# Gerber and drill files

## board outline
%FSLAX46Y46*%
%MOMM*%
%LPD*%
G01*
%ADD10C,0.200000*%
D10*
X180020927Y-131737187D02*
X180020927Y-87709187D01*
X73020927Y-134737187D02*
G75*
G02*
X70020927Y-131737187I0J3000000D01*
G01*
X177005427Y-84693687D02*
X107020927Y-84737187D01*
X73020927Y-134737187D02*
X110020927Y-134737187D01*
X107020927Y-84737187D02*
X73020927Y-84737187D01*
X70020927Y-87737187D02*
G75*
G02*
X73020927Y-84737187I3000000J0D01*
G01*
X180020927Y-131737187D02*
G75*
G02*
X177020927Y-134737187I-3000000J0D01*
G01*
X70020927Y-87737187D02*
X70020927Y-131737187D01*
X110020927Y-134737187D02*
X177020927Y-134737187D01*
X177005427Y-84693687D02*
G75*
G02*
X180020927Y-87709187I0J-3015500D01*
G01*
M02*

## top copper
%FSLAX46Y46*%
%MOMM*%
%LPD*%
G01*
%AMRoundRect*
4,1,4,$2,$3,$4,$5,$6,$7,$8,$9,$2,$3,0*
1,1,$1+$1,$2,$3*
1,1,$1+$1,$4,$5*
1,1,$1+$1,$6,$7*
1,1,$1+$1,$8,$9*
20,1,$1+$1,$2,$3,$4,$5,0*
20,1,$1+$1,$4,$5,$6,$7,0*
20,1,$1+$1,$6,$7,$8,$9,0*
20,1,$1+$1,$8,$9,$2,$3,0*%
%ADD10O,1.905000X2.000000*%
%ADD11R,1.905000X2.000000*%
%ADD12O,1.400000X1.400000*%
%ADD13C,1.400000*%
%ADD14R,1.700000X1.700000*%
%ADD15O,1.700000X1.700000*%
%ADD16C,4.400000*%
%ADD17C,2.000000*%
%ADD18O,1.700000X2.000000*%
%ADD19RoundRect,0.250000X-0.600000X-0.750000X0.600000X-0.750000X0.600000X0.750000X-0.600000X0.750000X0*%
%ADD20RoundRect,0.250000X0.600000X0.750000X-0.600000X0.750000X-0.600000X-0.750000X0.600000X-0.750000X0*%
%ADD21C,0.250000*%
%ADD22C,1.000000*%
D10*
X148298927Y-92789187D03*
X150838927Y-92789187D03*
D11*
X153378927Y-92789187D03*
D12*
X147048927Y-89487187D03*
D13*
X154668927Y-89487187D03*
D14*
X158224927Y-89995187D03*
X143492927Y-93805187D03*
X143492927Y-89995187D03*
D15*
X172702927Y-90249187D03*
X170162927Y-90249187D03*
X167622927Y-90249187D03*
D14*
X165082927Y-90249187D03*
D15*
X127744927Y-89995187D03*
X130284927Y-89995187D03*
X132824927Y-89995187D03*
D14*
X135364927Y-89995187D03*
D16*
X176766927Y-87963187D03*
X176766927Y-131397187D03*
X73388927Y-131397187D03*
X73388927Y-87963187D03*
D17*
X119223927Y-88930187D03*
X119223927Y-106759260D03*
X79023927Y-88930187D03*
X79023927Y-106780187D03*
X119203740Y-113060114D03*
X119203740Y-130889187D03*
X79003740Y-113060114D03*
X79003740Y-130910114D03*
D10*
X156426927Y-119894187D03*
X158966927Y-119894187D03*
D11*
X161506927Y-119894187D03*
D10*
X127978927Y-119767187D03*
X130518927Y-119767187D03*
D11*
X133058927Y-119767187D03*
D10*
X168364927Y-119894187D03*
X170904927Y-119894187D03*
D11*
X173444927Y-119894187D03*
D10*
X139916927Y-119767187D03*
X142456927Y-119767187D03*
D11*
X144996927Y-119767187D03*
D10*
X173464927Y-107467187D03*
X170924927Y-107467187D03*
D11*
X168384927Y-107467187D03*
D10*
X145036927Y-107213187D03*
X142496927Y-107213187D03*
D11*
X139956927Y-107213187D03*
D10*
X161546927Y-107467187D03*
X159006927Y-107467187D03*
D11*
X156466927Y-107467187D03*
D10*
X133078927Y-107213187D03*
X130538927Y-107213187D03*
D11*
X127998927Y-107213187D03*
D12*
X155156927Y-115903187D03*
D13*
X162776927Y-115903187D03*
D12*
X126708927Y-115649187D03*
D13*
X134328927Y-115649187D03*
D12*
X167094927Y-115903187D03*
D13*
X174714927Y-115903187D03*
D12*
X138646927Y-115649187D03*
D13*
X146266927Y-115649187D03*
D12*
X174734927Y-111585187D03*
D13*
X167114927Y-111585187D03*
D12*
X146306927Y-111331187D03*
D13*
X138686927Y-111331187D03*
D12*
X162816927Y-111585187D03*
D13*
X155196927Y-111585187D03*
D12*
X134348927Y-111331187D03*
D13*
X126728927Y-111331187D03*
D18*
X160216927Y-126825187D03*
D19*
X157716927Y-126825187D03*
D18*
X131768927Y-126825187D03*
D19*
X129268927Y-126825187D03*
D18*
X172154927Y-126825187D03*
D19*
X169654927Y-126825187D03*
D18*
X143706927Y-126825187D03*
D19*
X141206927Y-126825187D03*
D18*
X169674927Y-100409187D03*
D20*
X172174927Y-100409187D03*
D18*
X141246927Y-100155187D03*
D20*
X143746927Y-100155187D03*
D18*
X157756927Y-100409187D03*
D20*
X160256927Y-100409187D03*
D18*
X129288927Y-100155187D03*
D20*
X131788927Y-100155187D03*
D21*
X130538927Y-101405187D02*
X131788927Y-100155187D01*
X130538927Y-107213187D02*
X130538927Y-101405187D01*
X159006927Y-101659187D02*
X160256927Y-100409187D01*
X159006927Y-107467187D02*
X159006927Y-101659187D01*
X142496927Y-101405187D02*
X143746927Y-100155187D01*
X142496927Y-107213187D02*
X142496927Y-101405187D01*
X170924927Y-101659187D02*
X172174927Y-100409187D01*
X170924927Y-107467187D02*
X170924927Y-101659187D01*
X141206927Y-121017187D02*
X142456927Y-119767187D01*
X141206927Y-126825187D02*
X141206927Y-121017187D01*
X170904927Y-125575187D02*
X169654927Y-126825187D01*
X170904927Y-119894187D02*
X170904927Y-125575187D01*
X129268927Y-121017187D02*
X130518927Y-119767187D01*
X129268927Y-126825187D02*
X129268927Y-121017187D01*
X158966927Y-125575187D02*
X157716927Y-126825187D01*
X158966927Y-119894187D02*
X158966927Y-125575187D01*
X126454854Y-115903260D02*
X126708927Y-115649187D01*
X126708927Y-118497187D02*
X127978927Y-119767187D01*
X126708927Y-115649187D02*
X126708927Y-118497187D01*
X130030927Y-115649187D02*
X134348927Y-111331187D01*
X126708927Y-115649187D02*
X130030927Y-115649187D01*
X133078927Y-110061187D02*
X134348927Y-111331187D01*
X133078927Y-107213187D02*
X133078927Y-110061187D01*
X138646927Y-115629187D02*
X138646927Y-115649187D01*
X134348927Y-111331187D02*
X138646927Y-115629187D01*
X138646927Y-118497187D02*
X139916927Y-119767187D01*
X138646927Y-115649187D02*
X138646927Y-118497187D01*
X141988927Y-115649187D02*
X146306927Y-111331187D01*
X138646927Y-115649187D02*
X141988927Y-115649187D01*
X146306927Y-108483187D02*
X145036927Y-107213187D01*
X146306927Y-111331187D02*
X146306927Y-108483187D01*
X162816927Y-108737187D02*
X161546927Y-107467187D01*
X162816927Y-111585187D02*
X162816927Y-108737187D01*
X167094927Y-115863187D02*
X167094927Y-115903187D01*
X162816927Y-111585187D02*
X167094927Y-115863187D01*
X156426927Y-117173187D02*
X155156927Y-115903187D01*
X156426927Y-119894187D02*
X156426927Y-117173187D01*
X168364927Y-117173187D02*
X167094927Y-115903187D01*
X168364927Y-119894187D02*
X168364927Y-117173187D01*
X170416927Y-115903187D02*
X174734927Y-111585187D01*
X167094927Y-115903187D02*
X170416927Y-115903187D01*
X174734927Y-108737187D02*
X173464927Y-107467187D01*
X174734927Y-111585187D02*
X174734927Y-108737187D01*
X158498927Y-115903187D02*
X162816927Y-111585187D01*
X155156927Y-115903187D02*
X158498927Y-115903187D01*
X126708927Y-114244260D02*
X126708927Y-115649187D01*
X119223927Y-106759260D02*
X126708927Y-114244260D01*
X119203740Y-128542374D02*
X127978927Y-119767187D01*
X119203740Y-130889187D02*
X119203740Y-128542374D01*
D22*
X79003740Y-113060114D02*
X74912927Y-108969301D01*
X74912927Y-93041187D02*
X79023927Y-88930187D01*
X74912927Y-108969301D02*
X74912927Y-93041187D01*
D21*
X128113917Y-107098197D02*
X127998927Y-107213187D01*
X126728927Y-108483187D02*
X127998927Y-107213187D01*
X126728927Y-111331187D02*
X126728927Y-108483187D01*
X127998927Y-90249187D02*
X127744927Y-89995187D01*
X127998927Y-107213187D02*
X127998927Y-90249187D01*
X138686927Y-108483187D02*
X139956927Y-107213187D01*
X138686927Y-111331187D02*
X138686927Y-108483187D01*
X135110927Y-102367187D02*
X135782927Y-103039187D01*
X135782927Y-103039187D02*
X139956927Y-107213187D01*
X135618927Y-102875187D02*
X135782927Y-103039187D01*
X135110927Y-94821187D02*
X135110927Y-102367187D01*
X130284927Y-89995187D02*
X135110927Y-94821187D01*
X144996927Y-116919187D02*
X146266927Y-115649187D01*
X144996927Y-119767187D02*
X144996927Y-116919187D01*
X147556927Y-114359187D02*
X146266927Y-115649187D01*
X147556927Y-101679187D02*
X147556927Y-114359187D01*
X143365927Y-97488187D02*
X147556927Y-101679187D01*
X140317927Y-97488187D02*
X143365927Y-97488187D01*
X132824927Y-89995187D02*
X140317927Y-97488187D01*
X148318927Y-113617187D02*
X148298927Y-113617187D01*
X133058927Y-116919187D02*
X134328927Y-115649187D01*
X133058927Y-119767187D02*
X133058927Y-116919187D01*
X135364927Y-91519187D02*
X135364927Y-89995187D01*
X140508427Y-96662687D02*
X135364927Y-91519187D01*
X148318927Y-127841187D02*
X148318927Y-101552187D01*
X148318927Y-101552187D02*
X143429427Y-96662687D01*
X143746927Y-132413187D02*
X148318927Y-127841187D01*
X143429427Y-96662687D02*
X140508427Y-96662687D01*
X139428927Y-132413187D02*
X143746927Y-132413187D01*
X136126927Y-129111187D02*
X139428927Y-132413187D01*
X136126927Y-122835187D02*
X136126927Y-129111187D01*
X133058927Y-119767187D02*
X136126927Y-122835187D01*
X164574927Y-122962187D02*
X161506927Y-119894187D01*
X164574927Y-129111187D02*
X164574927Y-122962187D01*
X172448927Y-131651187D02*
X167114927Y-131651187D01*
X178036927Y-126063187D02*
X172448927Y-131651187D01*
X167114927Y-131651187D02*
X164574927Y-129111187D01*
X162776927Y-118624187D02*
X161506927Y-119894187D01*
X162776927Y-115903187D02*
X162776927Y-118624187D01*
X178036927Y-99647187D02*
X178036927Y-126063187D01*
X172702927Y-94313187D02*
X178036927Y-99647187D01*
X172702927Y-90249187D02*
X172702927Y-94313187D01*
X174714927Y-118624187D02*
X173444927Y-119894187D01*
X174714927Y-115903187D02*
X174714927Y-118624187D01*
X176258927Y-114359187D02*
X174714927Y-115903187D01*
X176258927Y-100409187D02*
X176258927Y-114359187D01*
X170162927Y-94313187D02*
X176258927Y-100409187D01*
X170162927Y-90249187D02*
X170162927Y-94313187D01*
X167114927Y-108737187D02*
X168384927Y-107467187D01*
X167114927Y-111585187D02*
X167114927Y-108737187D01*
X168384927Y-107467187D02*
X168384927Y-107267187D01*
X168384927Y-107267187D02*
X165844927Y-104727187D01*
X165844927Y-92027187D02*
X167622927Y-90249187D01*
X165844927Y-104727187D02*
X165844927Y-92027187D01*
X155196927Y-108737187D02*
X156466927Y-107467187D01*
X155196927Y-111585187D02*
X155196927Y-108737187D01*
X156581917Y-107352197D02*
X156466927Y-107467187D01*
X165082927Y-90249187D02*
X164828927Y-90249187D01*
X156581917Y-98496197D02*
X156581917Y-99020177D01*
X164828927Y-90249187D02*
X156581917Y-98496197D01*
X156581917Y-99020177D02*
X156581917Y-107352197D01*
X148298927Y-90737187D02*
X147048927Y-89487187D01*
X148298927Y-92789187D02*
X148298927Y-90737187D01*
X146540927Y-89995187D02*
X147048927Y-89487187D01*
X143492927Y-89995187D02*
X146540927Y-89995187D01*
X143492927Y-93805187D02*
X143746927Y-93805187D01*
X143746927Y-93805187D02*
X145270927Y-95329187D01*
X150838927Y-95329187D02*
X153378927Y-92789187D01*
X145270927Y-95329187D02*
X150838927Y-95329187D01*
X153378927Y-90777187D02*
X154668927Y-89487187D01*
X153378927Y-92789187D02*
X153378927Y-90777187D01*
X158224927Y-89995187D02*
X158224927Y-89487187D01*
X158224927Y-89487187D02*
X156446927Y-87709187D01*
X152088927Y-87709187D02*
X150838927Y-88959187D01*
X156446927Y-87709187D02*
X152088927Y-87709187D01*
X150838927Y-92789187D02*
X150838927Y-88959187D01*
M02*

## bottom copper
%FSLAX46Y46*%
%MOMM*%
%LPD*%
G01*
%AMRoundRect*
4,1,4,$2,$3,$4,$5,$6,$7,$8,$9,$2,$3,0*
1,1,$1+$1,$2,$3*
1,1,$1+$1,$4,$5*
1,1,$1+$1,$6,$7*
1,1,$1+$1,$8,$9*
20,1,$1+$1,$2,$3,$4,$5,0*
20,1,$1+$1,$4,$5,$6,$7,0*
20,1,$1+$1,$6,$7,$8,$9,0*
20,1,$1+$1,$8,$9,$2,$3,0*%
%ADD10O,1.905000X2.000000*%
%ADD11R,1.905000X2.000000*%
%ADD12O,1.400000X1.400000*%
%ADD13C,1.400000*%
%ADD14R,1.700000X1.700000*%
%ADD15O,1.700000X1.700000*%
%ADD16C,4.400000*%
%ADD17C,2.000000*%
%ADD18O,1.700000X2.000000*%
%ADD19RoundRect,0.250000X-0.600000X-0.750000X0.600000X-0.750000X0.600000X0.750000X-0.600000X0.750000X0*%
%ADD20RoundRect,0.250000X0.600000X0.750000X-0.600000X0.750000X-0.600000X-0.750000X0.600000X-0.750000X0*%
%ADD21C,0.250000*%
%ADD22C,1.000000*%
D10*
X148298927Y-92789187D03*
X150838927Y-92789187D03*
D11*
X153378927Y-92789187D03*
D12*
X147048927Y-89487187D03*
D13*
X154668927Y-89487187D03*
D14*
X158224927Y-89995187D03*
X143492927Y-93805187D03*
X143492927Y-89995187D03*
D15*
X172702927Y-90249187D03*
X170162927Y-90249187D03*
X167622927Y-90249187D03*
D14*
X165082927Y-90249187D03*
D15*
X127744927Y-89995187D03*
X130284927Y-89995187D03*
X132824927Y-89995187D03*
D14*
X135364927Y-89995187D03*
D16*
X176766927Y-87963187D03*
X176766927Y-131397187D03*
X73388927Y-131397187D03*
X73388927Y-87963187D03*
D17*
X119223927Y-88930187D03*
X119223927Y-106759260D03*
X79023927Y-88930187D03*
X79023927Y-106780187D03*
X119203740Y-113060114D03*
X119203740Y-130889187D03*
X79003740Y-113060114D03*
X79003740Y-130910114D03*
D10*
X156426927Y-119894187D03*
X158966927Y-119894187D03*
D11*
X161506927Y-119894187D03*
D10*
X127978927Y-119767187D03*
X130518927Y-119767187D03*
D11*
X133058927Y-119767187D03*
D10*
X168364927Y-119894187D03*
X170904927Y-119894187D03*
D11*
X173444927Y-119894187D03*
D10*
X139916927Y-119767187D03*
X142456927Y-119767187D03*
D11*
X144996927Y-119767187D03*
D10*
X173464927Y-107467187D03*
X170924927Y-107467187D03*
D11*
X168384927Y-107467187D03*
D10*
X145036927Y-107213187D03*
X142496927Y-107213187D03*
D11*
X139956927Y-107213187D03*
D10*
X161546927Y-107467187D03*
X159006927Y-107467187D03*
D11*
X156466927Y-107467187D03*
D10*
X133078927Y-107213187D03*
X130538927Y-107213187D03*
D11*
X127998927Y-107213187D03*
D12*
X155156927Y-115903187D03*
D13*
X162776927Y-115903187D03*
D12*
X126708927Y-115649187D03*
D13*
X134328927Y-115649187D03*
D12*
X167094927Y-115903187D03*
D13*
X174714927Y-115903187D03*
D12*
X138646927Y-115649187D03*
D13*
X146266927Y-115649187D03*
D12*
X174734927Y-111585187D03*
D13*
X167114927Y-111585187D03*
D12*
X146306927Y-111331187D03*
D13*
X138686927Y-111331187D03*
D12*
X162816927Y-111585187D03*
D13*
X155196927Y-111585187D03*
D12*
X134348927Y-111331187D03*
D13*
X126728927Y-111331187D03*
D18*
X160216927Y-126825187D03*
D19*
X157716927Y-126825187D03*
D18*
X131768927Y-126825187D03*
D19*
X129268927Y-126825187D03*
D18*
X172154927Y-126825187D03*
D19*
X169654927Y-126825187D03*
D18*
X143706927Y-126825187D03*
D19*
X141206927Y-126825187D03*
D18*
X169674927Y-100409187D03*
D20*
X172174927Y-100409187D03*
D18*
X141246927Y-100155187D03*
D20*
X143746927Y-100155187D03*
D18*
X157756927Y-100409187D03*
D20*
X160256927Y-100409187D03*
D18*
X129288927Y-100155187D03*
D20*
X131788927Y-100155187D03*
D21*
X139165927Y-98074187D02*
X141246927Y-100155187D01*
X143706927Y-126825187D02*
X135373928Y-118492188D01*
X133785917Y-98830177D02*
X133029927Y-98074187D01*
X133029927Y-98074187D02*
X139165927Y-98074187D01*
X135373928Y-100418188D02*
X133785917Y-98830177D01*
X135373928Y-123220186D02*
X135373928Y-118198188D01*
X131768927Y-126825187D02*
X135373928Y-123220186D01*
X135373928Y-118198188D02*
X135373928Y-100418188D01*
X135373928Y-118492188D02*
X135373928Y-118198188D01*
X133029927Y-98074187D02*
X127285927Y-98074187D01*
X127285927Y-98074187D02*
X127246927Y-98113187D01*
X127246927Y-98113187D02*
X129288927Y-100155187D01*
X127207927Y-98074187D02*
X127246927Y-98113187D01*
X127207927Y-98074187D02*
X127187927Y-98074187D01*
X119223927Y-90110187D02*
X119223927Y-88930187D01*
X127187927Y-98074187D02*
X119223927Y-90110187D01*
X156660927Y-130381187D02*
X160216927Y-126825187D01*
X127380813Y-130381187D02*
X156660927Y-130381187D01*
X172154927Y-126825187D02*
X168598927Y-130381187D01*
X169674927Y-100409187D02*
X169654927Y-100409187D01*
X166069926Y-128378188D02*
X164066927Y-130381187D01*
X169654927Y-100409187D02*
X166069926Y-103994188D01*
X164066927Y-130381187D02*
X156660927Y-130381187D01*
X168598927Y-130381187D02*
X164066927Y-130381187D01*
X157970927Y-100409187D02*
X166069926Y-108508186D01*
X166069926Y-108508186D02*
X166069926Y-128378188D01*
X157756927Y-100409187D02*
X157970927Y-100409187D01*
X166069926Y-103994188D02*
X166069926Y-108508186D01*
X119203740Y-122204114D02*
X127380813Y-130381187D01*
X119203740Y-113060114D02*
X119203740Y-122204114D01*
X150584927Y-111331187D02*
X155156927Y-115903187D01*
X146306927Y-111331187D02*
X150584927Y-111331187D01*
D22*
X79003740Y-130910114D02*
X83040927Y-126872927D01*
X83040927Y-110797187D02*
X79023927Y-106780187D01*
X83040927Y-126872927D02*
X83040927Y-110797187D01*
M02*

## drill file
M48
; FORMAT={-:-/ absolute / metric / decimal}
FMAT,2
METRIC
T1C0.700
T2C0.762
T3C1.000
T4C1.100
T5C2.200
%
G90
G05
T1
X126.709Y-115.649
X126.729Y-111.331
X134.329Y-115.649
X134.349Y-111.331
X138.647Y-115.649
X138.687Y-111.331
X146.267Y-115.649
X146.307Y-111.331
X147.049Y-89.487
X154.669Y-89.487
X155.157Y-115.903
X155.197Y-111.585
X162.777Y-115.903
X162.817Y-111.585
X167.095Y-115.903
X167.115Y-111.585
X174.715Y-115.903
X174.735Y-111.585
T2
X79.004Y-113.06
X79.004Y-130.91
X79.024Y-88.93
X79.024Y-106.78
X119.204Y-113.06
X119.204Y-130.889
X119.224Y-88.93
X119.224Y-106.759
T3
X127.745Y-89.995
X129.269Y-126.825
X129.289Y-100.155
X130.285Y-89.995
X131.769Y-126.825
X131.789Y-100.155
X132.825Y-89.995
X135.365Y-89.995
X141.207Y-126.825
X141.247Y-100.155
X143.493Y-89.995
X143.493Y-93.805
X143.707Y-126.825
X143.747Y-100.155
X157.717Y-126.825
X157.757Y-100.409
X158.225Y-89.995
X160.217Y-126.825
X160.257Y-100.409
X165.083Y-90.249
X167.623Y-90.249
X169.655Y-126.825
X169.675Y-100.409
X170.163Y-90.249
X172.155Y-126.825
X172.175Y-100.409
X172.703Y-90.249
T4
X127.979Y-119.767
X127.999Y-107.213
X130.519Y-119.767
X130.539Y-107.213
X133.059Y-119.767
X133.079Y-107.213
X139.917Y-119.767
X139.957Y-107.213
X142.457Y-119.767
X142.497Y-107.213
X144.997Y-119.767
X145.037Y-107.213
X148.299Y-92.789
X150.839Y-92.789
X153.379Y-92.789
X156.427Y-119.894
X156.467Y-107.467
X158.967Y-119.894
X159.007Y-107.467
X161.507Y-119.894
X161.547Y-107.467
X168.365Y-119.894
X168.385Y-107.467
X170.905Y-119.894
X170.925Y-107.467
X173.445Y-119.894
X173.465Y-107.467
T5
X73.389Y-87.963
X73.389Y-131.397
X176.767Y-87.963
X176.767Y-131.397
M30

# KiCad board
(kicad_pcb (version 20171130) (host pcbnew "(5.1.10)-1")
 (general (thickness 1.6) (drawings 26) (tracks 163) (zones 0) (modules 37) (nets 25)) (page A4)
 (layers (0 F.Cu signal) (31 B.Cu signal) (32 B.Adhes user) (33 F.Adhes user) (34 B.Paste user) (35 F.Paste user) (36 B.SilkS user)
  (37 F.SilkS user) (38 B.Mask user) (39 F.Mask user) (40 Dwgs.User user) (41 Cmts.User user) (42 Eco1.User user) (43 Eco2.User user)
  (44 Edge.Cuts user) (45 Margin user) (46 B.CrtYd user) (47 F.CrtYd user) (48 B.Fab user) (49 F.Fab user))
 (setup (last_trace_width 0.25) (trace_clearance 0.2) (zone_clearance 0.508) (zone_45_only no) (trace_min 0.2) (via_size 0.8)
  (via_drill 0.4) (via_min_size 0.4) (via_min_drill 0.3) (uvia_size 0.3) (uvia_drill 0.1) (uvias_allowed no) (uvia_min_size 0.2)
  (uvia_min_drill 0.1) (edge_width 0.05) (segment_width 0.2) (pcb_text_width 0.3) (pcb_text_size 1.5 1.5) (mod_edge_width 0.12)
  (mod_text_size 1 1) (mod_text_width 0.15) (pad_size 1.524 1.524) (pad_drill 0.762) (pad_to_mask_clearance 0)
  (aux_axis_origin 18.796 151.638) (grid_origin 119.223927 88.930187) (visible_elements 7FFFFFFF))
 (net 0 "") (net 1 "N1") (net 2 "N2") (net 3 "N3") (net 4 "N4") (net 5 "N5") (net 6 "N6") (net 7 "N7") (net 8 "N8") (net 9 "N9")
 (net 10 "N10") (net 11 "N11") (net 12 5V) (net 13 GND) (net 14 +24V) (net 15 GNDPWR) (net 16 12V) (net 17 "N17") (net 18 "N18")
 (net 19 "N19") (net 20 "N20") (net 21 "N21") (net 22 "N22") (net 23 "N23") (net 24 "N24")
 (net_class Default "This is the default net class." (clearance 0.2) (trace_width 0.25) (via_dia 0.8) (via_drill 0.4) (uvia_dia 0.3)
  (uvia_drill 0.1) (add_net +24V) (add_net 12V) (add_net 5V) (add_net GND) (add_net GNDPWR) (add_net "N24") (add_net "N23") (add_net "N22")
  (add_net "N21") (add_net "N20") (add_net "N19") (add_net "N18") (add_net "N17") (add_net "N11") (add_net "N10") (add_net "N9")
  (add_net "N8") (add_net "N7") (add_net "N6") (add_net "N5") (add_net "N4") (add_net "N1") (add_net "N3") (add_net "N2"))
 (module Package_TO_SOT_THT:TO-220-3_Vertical (layer F.Cu) (at 153.378927 92.789187 180)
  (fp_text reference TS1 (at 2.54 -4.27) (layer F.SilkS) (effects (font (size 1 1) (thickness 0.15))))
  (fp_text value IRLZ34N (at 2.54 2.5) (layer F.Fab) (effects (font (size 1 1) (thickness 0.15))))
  (pad 3 thru_hole oval (at 5.08 0 180) (size 1.905 2) (drill 1.1) (layers *.Cu *.Mask) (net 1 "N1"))
  (pad 2 thru_hole oval (at 2.54 0 180) (size 1.905 2) (drill 1.1) (layers *.Cu *.Mask) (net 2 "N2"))
  (pad 1 thru_hole rect (at 0 0 180) (size 1.905 2) (drill 1.1) (layers *.Cu *.Mask) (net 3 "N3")))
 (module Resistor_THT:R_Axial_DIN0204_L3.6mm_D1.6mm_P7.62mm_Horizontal (layer F.Cu) (at 154.668927 89.487187 180)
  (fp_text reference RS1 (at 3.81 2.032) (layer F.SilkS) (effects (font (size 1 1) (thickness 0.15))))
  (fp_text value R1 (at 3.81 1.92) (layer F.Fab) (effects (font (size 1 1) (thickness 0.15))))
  (pad 2 thru_hole oval (at 7.62 0 180) (size 1.4 1.4) (drill 0.7) (layers *.Cu *.Mask) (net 1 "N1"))
  (pad 1 thru_hole circle (at 0 0 180) (size 1.4 1.4) (drill 0.7) (layers *.Cu *.Mask) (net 3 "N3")))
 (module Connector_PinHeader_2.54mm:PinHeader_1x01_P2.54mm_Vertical (layer F.Cu) (at 158.224927 89.995187 180)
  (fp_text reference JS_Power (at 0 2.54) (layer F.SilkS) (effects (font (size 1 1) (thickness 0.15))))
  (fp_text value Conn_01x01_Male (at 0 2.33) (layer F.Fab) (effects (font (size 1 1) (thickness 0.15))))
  (pad 1 thru_hole rect (at 0 0 180) (size 1.7 1.7) (drill 1) (layers *.Cu *.Mask) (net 2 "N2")))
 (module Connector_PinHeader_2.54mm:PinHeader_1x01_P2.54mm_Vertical (layer F.Cu) (at 143.492927 93.805187 180)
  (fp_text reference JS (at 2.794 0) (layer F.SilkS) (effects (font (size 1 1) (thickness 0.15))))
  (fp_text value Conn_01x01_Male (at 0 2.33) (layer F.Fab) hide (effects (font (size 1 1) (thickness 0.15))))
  (pad 1 thru_hole rect (at 0 0 180) (size 1.7 1.7) (drill 1) (layers *.Cu *.Mask) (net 3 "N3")))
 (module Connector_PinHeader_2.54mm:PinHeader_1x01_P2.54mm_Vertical (layer F.Cu) (at 143.492927 89.995187 180)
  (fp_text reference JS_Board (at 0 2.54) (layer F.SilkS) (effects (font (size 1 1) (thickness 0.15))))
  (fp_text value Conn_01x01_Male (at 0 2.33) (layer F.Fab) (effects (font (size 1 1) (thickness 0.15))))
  (pad 1 thru_hole rect (at 0 0 180) (size 1.7 1.7) (drill 1) (layers *.Cu *.Mask) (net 1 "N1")))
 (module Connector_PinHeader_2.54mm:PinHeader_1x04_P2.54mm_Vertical (layer F.Cu) (at 165.082927 90.249187 90)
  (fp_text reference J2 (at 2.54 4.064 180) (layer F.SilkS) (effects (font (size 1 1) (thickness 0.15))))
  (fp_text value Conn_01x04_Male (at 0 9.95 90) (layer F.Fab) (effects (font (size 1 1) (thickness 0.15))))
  (pad 4 thru_hole oval (at 0 7.62 90) (size 1.7 1.7) (drill 1) (layers *.Cu *.Mask) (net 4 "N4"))
  (pad 3 thru_hole oval (at 0 5.08 90) (size 1.7 1.7) (drill 1) (layers *.Cu *.Mask) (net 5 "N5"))
  (pad 2 thru_hole oval (at 0 2.54 90) (size 1.7 1.7) (drill 1) (layers *.Cu *.Mask) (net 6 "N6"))
  (pad 1 thru_hole rect (at 0 0 90) (size 1.7 1.7) (drill 1) (layers *.Cu *.Mask) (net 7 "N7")))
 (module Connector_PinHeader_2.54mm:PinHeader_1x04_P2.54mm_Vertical (layer F.Cu) (at 135.364927 89.995187 270)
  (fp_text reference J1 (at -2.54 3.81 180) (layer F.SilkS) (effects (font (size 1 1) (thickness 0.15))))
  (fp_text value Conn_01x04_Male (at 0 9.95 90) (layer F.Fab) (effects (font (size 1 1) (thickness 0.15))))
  (pad 4 thru_hole oval (at 0 7.62 270) (size 1.7 1.7) (drill 1) (layers *.Cu *.Mask) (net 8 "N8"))
  (pad 3 thru_hole oval (at 0 5.08 270) (size 1.7 1.7) (drill 1) (layers *.Cu *.Mask) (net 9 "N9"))
  (pad 2 thru_hole oval (at 0 2.54 270) (size 1.7 1.7) (drill 1) (layers *.Cu *.Mask) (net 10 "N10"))
  (pad 1 thru_hole rect (at 0 0 270) (size 1.7 1.7) (drill 1) (layers *.Cu *.Mask) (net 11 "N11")))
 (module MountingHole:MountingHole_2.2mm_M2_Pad (layer F.Cu) (at 176.766927 87.963187)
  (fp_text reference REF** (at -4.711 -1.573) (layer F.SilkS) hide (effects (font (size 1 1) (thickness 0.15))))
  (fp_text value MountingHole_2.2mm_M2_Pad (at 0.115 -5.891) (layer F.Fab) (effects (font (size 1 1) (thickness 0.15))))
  (pad 1 thru_hole circle (at 0 0) (size 4.4 4.4) (drill 2.2) (layers *.Cu *.Mask)))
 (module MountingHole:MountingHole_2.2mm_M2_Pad (layer F.Cu) (at 176.766927 131.397187)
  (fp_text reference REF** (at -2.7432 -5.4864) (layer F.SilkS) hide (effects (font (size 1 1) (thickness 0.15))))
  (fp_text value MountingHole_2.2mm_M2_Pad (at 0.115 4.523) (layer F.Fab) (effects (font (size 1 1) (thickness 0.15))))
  (pad 1 thru_hole circle (at 0 0) (size 4.4 4.4) (drill 2.2) (layers *.Cu *.Mask)))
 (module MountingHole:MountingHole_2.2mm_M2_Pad (layer F.Cu) (at 73.388927 131.397187)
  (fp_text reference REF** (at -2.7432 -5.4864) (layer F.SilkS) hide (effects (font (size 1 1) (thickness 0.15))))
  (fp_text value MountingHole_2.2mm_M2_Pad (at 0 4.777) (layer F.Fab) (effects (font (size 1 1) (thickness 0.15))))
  (pad 1 thru_hole circle (at 0 0) (size 4.4 4.4) (drill 2.2) (layers *.Cu *.Mask)))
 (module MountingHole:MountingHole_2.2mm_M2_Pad (layer F.Cu) (at 73.388927 87.963187)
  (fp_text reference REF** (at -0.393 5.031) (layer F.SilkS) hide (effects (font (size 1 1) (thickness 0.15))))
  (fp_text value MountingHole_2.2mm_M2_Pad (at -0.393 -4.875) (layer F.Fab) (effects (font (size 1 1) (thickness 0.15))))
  (pad 1 thru_hole circle (at 0 0) (size 4.4 4.4) (drill 2.2) (layers *.Cu *.Mask)))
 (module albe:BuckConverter (layer F.Cu) (at 99.825114 97.86926 270)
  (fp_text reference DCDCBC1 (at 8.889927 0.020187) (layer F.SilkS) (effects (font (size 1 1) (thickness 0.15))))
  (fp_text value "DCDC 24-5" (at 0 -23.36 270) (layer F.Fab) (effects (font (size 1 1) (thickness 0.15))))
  (pad 4 thru_hole circle (at -8.939073 -19.398813 270) (size 2 2) (drill 0.762) (layers *.Cu *.Mask) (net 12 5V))
  (pad 3 thru_hole circle (at 8.89 -19.398813 270) (size 2 2) (drill 0.762) (layers *.Cu *.Mask) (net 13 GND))
  (pad 2 thru_hole circle (at -8.939073 20.801187 270) (size 2 2) (drill 0.762) (layers *.Cu *.Mask) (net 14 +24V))
  (pad 1 thru_hole circle (at 8.910927 20.801187 270) (size 2 2) (drill 0.762) (layers *.Cu *.Mask) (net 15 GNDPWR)))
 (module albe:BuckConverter (layer F.Cu) (at 99.804927 121.999187 270)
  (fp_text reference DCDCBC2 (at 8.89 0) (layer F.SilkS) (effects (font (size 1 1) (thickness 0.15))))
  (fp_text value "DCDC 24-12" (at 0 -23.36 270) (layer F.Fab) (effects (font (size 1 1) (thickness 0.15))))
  (pad 4 thru_hole circle (at -8.939073 -19.398813 270) (size 2 2) (drill 0.762) (layers *.Cu *.Mask) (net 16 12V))
  (pad 3 thru_hole circle (at 8.89 -19.398813 270) (size 2 2) (drill 0.762) (layers *.Cu *.Mask) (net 13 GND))
  (pad 2 thru_hole circle (at -8.939073 20.801187 270) (size 2 2) (drill 0.762) (layers *.Cu *.Mask) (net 14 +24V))
  (pad 1 thru_hole circle (at 8.910927 20.801187 270) (size 2 2) (drill 0.762) (layers *.Cu *.Mask) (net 15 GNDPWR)))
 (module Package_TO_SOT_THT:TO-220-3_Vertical (layer F.Cu) (at 161.506927 119.894187 180)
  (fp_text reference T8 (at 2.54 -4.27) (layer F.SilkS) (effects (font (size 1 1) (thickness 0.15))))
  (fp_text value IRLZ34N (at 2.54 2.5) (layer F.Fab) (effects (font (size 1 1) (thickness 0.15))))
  (pad 3 thru_hole oval (at 5.08 0 180) (size 1.905 2) (drill 1.1) (layers *.Cu *.Mask) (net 13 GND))
  (pad 2 thru_hole oval (at 2.54 0 180) (size 1.905 2) (drill 1.1) (layers *.Cu *.Mask) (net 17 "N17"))
  (pad 1 thru_hole rect (at 0 0 180) (size 1.905 2) (drill 1.1) (layers *.Cu *.Mask) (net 4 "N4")))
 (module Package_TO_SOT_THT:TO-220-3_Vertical (layer F.Cu) (at 133.058927 119.767187 180)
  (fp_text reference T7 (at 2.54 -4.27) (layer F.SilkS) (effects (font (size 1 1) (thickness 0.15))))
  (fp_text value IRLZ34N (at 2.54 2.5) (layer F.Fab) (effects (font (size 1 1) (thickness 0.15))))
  (pad 3 thru_hole oval (at 5.08 0 180) (size 1.905 2) (drill 1.1) (layers *.Cu *.Mask) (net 13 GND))
  (pad 2 thru_hole oval (at 2.54 0 180) (size 1.905 2) (drill 1.1) (layers *.Cu *.Mask) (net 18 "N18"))
  (pad 1 thru_hole rect (at 0 0 180) (size 1.905 2) (drill 1.1) (layers *.Cu *.Mask) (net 11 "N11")))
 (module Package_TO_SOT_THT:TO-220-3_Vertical (layer F.Cu) (at 173.444927 119.894187 180)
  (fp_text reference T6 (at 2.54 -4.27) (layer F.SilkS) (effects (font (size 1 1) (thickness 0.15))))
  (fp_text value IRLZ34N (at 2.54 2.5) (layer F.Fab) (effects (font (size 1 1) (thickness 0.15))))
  (pad 3 thru_hole oval (at 5.08 0 180) (size 1.905 2) (drill 1.1) (layers *.Cu *.Mask) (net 13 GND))
  (pad 2 thru_hole oval (at 2.54 0 180) (size 1.905 2) (drill 1.1) (layers *.Cu *.Mask) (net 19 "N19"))
  (pad 1 thru_hole rect (at 0 0 180) (size 1.905 2) (drill 1.1) (layers *.Cu *.Mask) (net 5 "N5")))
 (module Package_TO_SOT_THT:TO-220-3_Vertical (layer F.Cu) (at 144.996927 119.767187 180)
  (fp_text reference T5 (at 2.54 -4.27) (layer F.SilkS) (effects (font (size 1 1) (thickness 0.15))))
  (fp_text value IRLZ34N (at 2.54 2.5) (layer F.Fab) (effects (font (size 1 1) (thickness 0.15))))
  (pad 3 thru_hole oval (at 5.08 0 180) (size 1.905 2) (drill 1.1) (layers *.Cu *.Mask) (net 13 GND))
  (pad 2 thru_hole oval (at 2.54 0 180) (size 1.905 2) (drill 1.1) (layers *.Cu *.Mask) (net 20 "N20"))
  (pad 1 thru_hole rect (at 0 0 180) (size 1.905 2) (drill 1.1) (layers *.Cu *.Mask) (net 10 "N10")))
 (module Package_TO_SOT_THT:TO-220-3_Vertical (layer F.Cu) (at 168.384927 107.467187)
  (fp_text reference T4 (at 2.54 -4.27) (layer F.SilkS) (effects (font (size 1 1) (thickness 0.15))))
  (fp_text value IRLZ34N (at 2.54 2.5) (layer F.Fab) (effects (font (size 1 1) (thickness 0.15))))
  (pad 3 thru_hole oval (at 5.08 0) (size 1.905 2) (drill 1.1) (layers *.Cu *.Mask) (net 13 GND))
  (pad 2 thru_hole oval (at 2.54 0) (size 1.905 2) (drill 1.1) (layers *.Cu *.Mask) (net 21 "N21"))
  (pad 1 thru_hole rect (at 0 0) (size 1.905 2) (drill 1.1) (layers *.Cu *.Mask) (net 6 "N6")))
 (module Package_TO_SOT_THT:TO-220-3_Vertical (layer F.Cu) (at 139.956927 107.213187)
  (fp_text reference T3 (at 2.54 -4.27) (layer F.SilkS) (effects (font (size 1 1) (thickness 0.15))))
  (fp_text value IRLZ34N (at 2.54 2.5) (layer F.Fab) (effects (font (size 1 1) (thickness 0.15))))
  (pad 3 thru_hole oval (at 5.08 0) (size 1.905 2) (drill 1.1) (layers *.Cu *.Mask) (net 13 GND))
  (pad 2 thru_hole oval (at 2.54 0) (size 1.905 2) (drill 1.1) (layers *.Cu *.Mask) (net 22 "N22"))
  (pad 1 thru_hole rect (at 0 0) (size 1.905 2) (drill 1.1) (layers *.Cu *.Mask) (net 9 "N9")))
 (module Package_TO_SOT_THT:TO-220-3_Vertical (layer F.Cu) (at 156.466927 107.467187)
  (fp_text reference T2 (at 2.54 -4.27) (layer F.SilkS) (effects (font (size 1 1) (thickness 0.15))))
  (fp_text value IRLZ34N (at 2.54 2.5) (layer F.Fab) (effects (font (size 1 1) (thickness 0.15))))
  (pad 3 thru_hole oval (at 5.08 0) (size 1.905 2) (drill 1.1) (layers *.Cu *.Mask) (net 13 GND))
  (pad 2 thru_hole oval (at 2.54 0) (size 1.905 2) (drill 1.1) (layers *.Cu *.Mask) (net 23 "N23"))
  (pad 1 thru_hole rect (at 0 0) (size 1.905 2) (drill 1.1) (layers *.Cu *.Mask) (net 7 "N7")))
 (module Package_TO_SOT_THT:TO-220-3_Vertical (layer F.Cu) (at 127.998927 107.213187)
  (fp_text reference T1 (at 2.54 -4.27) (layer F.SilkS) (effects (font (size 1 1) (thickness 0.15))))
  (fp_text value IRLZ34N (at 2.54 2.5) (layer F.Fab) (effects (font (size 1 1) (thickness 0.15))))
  (pad 3 thru_hole oval (at 5.08 0) (size 1.905 2) (drill 1.1) (layers *.Cu *.Mask) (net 13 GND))
  (pad 2 thru_hole oval (at 2.54 0) (size 1.905 2) (drill 1.1) (layers *.Cu *.Mask) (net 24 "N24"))
  (pad 1 thru_hole rect (at 0 0) (size 1.905 2) (drill 1.1) (layers *.Cu *.Mask) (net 8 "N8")))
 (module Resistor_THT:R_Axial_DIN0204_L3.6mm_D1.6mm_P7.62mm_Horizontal (layer F.Cu) (at 162.776927 115.903187 180)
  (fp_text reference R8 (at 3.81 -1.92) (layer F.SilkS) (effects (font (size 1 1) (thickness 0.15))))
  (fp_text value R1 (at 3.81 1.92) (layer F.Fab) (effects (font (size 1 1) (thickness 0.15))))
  (pad 2 thru_hole oval (at 7.62 0 180) (size 1.4 1.4) (drill 0.7) (layers *.Cu *.Mask) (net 13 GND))
  (pad 1 thru_hole circle (at 0 0 180) (size 1.4 1.4) (drill 0.7) (layers *.Cu *.Mask) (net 4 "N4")))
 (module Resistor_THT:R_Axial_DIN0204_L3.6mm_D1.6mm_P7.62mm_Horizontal (layer F.Cu) (at 134.328927 115.649187 180)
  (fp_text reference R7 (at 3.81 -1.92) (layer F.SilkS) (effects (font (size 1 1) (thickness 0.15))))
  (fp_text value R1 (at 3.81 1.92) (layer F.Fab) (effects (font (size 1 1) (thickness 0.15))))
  (pad 2 thru_hole oval (at 7.62 0 180) (size 1.4 1.4) (drill 0.7) (layers *.Cu *.Mask) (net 13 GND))
  (pad 1 thru_hole circle (at 0 0 180) (size 1.4 1.4) (drill 0.7) (layers *.Cu *.Mask) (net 11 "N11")))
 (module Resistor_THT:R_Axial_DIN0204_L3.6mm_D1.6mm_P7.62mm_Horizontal (layer F.Cu) (at 174.714927 115.903187 180)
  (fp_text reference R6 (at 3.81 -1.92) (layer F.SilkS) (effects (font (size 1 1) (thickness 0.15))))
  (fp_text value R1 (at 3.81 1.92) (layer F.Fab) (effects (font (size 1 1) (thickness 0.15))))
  (pad 2 thru_hole oval (at 7.62 0 180) (size 1.4 1.4) (drill 0.7) (layers *.Cu *.Mask) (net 13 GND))
  (pad 1 thru_hole circle (at 0 0 180) (size 1.4 1.4) (drill 0.7) (layers *.Cu *.Mask) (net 5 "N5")))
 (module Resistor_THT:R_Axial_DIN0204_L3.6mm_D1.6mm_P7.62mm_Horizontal (layer F.Cu) (at 146.266927 115.649187 180)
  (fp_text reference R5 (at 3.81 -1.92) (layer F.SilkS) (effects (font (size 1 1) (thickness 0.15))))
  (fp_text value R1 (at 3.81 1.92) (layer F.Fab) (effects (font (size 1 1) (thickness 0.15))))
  (pad 2 thru_hole oval (at 7.62 0 180) (size 1.4 1.4) (drill 0.7) (layers *.Cu *.Mask) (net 13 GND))
  (pad 1 thru_hole circle (at 0 0 180) (size 1.4 1.4) (drill 0.7) (layers *.Cu *.Mask) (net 10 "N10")))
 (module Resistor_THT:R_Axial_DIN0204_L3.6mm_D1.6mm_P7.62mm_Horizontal (layer F.Cu) (at 167.114927 111.585187)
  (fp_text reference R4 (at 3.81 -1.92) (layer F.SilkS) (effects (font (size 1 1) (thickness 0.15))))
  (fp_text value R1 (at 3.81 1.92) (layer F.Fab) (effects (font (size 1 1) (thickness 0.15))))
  (pad 2 thru_hole oval (at 7.62 0) (size 1.4 1.4) (drill 0.7) (layers *.Cu *.Mask) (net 13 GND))
  (pad 1 thru_hole circle (at 0 0) (size 1.4 1.4) (drill 0.7) (layers *.Cu *.Mask) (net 6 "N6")))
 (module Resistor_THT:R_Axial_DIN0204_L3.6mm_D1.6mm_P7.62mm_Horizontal (layer F.Cu) (at 138.686927 111.331187)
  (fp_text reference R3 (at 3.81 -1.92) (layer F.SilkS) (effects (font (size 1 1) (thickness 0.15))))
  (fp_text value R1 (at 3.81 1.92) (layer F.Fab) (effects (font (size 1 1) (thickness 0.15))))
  (pad 2 thru_hole oval (at 7.62 0) (size 1.4 1.4) (drill 0.7) (layers *.Cu *.Mask) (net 13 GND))
  (pad 1 thru_hole circle (at 0 0) (size 1.4 1.4) (drill 0.7) (layers *.Cu *.Mask) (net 9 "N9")))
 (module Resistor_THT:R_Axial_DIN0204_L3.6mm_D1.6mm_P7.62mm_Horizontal (layer F.Cu) (at 155.196927 111.585187)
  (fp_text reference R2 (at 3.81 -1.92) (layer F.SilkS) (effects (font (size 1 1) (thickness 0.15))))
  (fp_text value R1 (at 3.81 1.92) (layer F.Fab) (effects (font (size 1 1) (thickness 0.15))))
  (pad 2 thru_hole oval (at 7.62 0) (size 1.4 1.4) (drill 0.7) (layers *.Cu *.Mask) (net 13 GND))
  (pad 1 thru_hole circle (at 0 0) (size 1.4 1.4) (drill 0.7) (layers *.Cu *.Mask) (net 7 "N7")))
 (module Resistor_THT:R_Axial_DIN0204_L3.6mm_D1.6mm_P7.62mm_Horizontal (layer F.Cu) (at 126.728927 111.331187)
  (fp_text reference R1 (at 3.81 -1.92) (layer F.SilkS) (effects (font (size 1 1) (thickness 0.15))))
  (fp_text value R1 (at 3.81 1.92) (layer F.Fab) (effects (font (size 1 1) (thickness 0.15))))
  (pad 2 thru_hole oval (at 7.62 0) (size 1.4 1.4) (drill 0.7) (layers *.Cu *.Mask) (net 13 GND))
  (pad 1 thru_hole circle (at 0 0) (size 1.4 1.4) (drill 0.7) (layers *.Cu *.Mask) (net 8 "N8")))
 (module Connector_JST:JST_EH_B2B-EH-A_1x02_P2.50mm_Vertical (layer F.Cu) (at 157.716927 126.825187)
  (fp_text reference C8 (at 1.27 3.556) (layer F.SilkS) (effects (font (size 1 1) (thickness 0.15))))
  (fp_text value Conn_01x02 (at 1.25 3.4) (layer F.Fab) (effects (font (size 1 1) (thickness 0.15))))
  (pad 2 thru_hole oval (at 2.5 0) (size 1.7 2) (drill 1) (layers *.Cu *.Mask) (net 16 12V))
  (pad 1 thru_hole roundrect (at 0 0) (size 1.7 2) (drill 1) (layers *.Cu *.Mask) (roundrect_rratio 0.1470588235294118) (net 17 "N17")))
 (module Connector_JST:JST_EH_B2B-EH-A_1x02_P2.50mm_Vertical (layer F.Cu) (at 129.268927 126.825187)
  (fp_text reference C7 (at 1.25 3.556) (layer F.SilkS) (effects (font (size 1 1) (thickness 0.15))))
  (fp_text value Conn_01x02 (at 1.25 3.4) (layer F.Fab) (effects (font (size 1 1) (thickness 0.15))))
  (pad 2 thru_hole oval (at 2.5 0) (size 1.7 2) (drill 1) (layers *.Cu *.Mask) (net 12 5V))
  (pad 1 thru_hole roundrect (at 0 0) (size 1.7 2) (drill 1) (layers *.Cu *.Mask) (roundrect_rratio 0.1470588235294118) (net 18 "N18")))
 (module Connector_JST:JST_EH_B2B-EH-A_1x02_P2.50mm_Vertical (layer F.Cu) (at 169.654927 126.825187)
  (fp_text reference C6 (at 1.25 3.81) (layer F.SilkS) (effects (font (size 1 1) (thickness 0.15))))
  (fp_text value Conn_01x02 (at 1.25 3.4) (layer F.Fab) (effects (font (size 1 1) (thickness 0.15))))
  (pad 2 thru_hole oval (at 2.5 0) (size 1.7 2) (drill 1) (layers *.Cu *.Mask) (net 16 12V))
  (pad 1 thru_hole roundrect (at 0 0) (size 1.7 2) (drill 1) (layers *.Cu *.Mask) (roundrect_rratio 0.1470588235294118) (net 19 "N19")))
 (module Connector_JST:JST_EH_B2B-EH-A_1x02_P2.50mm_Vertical (layer F.Cu) (at 141.206927 126.825187)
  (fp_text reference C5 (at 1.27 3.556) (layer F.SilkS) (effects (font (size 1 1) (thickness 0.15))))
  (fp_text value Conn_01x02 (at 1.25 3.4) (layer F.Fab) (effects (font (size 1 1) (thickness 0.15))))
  (pad 2 thru_hole oval (at 2.5 0) (size 1.7 2) (drill 1) (layers *.Cu *.Mask) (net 12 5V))
  (pad 1 thru_hole roundrect (at 0 0) (size 1.7 2) (drill 1) (layers *.Cu *.Mask) (roundrect_rratio 0.1470588235294118) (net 20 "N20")))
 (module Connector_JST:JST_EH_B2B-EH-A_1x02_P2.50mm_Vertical (layer F.Cu) (at 172.174927 100.409187 180)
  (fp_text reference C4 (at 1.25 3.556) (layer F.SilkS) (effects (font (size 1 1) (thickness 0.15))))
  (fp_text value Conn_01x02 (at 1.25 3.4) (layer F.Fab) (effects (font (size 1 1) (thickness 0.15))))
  (pad 2 thru_hole oval (at 2.5 0 180) (size 1.7 2) (drill 1) (layers *.Cu *.Mask) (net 16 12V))
  (pad 1 thru_hole roundrect (at 0 0 180) (size 1.7 2) (drill 1) (layers *.Cu *.Mask) (roundrect_rratio 0.1470588235294118) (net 21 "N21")))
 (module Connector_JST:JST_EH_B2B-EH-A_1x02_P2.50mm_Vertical (layer F.Cu) (at 143.746927 100.155187 180)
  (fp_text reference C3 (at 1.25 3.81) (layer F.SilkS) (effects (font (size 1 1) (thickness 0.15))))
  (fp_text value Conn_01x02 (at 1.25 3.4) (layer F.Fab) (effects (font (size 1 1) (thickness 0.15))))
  (pad 2 thru_hole oval (at 2.5 0 180) (size 1.7 2) (drill 1) (layers *.Cu *.Mask) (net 12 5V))
  (pad 1 thru_hole roundrect (at 0 0 180) (size 1.7 2) (drill 1) (layers *.Cu *.Mask) (roundrect_rratio 0.1470588235294118) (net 22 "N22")))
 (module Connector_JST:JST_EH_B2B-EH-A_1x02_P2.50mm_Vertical (layer F.Cu) (at 160.256927 100.409187 180)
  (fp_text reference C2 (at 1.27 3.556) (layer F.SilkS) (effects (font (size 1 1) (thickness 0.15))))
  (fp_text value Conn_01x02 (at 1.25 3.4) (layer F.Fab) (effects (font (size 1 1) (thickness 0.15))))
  (pad 2 thru_hole oval (at 2.5 0 180) (size 1.7 2) (drill 1) (layers *.Cu *.Mask) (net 16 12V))
  (pad 1 thru_hole roundrect (at 0 0 180) (size 1.7 2) (drill 1) (layers *.Cu *.Mask) (roundrect_rratio 0.1470588235294118) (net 23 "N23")))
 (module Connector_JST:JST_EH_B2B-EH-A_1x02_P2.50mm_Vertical (layer F.Cu) (at 131.788927 100.155187 180)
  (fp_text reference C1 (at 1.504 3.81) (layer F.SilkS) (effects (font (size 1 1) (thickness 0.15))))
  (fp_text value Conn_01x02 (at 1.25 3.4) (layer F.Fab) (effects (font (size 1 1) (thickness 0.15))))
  (pad 2 thru_hole oval (at 2.5 0 180) (size 1.7 2) (drill 1) (layers *.Cu *.Mask) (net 12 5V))
  (pad 1 thru_hole roundrect (at 0 0 180) (size 1.7 2) (drill 1) (layers *.Cu *.Mask) (roundrect_rratio 0.1470588235294118) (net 24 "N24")))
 (gr_line (start 180.020927 131.737187) (end 180.020927 87.709187) (layer Edge.Cuts) (width 0.2))
 (gr_arc (start 73.020927 131.737187) (end 70.020927 131.737187) (angle -90) (layer Edge.Cuts) (width 0.2))
 (gr_line (start 177.005427 84.693687) (end 107.020927 84.737187) (layer Edge.Cuts) (width 0.2))
 (gr_line (start 73.020927 134.737187) (end 110.020927 134.737187) (layer Edge.Cuts) (width 0.2))
 (gr_line (start 107.020927 84.737187) (end 73.020927 84.737187) (layer Edge.Cuts) (width 0.2))
 (gr_arc (start 73.020927 87.737187) (end 73.020927 84.737187) (angle -90) (layer Edge.Cuts) (width 0.2))
 (gr_arc (start 177.020927 131.737187) (end 177.020927 134.737187) (angle -90) (layer Edge.Cuts) (width 0.2))
 (gr_line (start 70.020927 87.737187) (end 70.020927 131.737187) (layer Edge.Cuts) (width 0.2))
 (gr_line (start 110.020927 134.737187) (end 177.020927 134.737187) (layer Edge.Cuts) (width 0.2))
 (gr_arc (start 177.005427 87.709187) (end 180.020927 87.709187) (angle -90) (layer Edge.Cuts) (width 0.2))
 (segment (start 139.165927 98.074187) (end 141.246927 100.155187) (width 0.25) (layer B.Cu) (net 12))
 (segment (start 143.706927 126.825187) (end 135.373928 118.492188) (width 0.25) (layer B.Cu) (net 12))
 (segment (start 133.785917 98.830177) (end 133.029927 98.074187) (width 0.25) (layer B.Cu) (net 12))
 (segment (start 133.029927 98.074187) (end 139.165927 98.074187) (width 0.25) (layer B.Cu) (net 12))
 (segment (start 135.373928 100.418188) (end 133.785917 98.830177) (width 0.25) (layer B.Cu) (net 12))
 (segment (start 135.373928 123.220186) (end 135.373928 118.198188) (width 0.25) (layer B.Cu) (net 12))
 (segment (start 131.768927 126.825187) (end 135.373928 123.220186) (width 0.25) (layer B.Cu) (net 12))
 (segment (start 135.373928 118.198188) (end 135.373928 100.418188) (width 0.25) (layer B.Cu) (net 12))
 (segment (start 135.373928 118.492188) (end 135.373928 118.198188) (width 0.25) (layer B.Cu) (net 12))
 (segment (start 133.029927 98.074187) (end 127.285927 98.074187) (width 0.25) (layer B.Cu) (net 12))
 (segment (start 127.285927 98.074187) (end 127.246927 98.113187) (width 0.25) (layer B.Cu) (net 12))
 (segment (start 127.246927 98.113187) (end 129.288927 100.155187) (width 0.25) (layer B.Cu) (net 12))
 (segment (start 127.207927 98.074187) (end 127.246927 98.113187) (width 0.25) (layer B.Cu) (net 12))
 (segment (start 127.207927 98.074187) (end 127.187927 98.074187) (width 0.25) (layer B.Cu) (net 12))
 (segment (start 119.223927 90.110187) (end 119.223927 88.930187) (width 0.25) (layer B.Cu) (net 12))
 (segment (start 127.187927 98.074187) (end 119.223927 90.110187) (width 0.25) (layer B.Cu) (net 12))
 (segment (start 130.538927 101.405187) (end 131.788927 100.155187) (width 0.25) (layer F.Cu) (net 24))
 (segment (start 130.538927 107.213187) (end 130.538927 101.405187) (width 0.25) (layer F.Cu) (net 24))
 (segment (start 156.660927 130.381187) (end 160.216927 126.825187) (width 0.25) (layer B.Cu) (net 16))
 (segment (start 127.380813 130.381187) (end 156.660927 130.381187) (width 0.25) (layer B.Cu) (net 16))
 (segment (start 172.154927 126.825187) (end 168.598927 130.381187) (width 0.25) (layer B.Cu) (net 16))
 (segment (start 169.674927 100.409187) (end 169.654927 100.409187) (width 0.25) (layer B.Cu) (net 16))
 (segment (start 166.069926 128.378188) (end 164.066927 130.381187) (width 0.25) (layer B.Cu) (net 16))
 (segment (start 169.654927 100.409187) (end 166.069926 103.994188) (width 0.25) (layer B.Cu) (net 16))
 (segment (start 164.066927 130.381187) (end 156.660927 130.381187) (width 0.25) (layer B.Cu) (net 16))
 (segment (start 168.598927 130.381187) (end 164.066927 130.381187) (width 0.25) (layer B.Cu) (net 16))
 (segment (start 157.970927 100.409187) (end 166.069926 108.508186) (width 0.25) (layer B.Cu) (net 16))
 (segment (start 166.069926 108.508186) (end 166.069926 128.378188) (width 0.25) (layer B.Cu) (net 16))
 (segment (start 157.756927 100.409187) (end 157.970927 100.409187) (width 0.25) (layer B.Cu) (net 16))
 (segment (start 166.069926 103.994188) (end 166.069926 108.508186) (width 0.25) (layer B.Cu) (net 16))
 (segment (start 119.20374 122.204114) (end 127.380813 130.381187) (width 0.25) (layer B.Cu) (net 16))
 (segment (start 119.20374 113.060114) (end 119.20374 122.204114) (width 0.25) (layer B.Cu) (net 16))
 (segment (start 159.006927 101.659187) (end 160.256927 100.409187) (width 0.25) (layer F.Cu) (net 23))
 (segment (start 159.006927 107.467187) (end 159.006927 101.659187) (width 0.25) (layer F.Cu) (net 23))
 (segment (start 142.496927 101.405187) (end 143.746927 100.155187) (width 0.25) (layer F.Cu) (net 22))
 (segment (start 142.496927 107.213187) (end 142.496927 101.405187) (width 0.25) (layer F.Cu) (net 22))
 (segment (start 170.924927 101.659187) (end 172.174927 100.409187) (width 0.25) (layer F.Cu) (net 21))
 (segment (start 170.924927 107.467187) (end 170.924927 101.659187) (width 0.25) (layer F.Cu) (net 21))
 (segment (start 141.206927 121.017187) (end 142.456927 119.767187) (width 0.25) (layer F.Cu) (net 20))
 (segment (start 141.206927 126.825187) (end 141.206927 121.017187) (width 0.25) (layer F.Cu) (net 20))
 (segment (start 170.904927 125.575187) (end 169.654927 126.825187) (width 0.25) (layer F.Cu) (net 19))
 (segment (start 170.904927 119.894187) (end 170.904927 125.575187) (width 0.25) (layer F.Cu) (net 19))
 (segment (start 129.268927 121.017187) (end 130.518927 119.767187) (width 0.25) (layer F.Cu) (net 18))
 (segment (start 129.268927 126.825187) (end 129.268927 121.017187) (width 0.25) (layer F.Cu) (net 18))
 (segment (start 158.966927 125.575187) (end 157.716927 126.825187) (width 0.25) (layer F.Cu) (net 17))
 (segment (start 158.966927 119.894187) (end 158.966927 125.575187) (width 0.25) (layer F.Cu) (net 17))
 (segment (start 126.454854 115.90326) (end 126.708927 115.649187) (width 0.25) (layer F.Cu) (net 13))
 (segment (start 126.708927 118.497187) (end 127.978927 119.767187) (width 0.25) (layer F.Cu) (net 13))
 (segment (start 126.708927 115.649187) (end 126.708927 118.497187) (width 0.25) (layer F.Cu) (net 13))
 (segment (start 130.030927 115.649187) (end 134.348927 111.331187) (width 0.25) (layer F.Cu) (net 13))
 (segment (start 126.708927 115.649187) (end 130.030927 115.649187) (width 0.25) (layer F.Cu) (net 13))
 (segment (start 133.078927 110.061187) (end 134.348927 111.331187) (width 0.25) (layer F.Cu) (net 13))
 (segment (start 133.078927 107.213187) (end 133.078927 110.061187) (width 0.25) (layer F.Cu) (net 13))
 (segment (start 138.646927 115.629187) (end 138.646927 115.649187) (width 0.25) (layer F.Cu) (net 13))
 (segment (start 134.348927 111.331187) (end 138.646927 115.629187) (width 0.25) (layer F.Cu) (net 13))
 (segment (start 138.646927 118.497187) (end 139.916927 119.767187) (width 0.25) (layer F.Cu) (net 13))
 (segment (start 138.646927 115.649187) (end 138.646927 118.497187) (width 0.25) (layer F.Cu) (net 13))
 (segment (start 141.988927 115.649187) (end 146.306927 111.331187) (width 0.25) (layer F.Cu) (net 13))
 (segment (start 138.646927 115.649187) (end 141.988927 115.649187) (width 0.25) (layer F.Cu) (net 13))
 (segment (start 146.306927 108.483187) (end 145.036927 107.213187) (width 0.25) (layer F.Cu) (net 13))
 (segment (start 146.306927 111.331187) (end 146.306927 108.483187) (width 0.25) (layer F.Cu) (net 13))
 (segment (start 162.816927 108.737187) (end 161.546927 107.467187) (width 0.25) (layer F.Cu) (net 13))
 (segment (start 162.816927 111.585187) (end 162.816927 108.737187) (width 0.25) (layer F.Cu) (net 13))
 (segment (start 167.094927 115.863187) (end 167.094927 115.903187) (width 0.25) (layer F.Cu) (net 13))
 (segment (start 162.816927 111.585187) (end 167.094927 115.863187) (width 0.25) (layer F.Cu) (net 13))
 (segment (start 156.426927 117.173187) (end 155.156927 115.903187) (width 0.25) (layer F.Cu) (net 13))
 (segment (start 156.426927 119.894187) (end 156.426927 117.173187) (width 0.25) (layer F.Cu) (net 13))
 (segment (start 168.364927 117.173187) (end 167.094927 115.903187) (width 0.25) (layer F.Cu) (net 13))
 (segment (start 168.364927 119.894187) (end 168.364927 117.173187) (width 0.25) (layer F.Cu) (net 13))
 (segment (start 170.416927 115.903187) (end 174.734927 111.585187) (width 0.25) (layer F.Cu) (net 13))
 (segment (start 167.094927 115.903187) (end 170.416927 115.903187) (width 0.25) (layer F.Cu) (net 13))
 (segment (start 174.734927 108.737187) (end 173.464927 107.467187) (width 0.25) (layer F.Cu) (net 13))
 (segment (start 174.734927 111.585187) (end 174.734927 108.737187) (width 0.25) (layer F.Cu) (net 13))
 (segment (start 158.498927 115.903187) (end 162.816927 111.585187) (width 0.25) (layer F.Cu) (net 13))
 (segment (start 155.156927 115.903187) (end 158.498927 115.903187) (width 0.25) (layer F.Cu) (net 13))
 (segment (start 150.584927 111.331187) (end 155.156927 115.903187) (width 0.25) (layer B.Cu) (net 13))
 (segment (start 146.306927 111.331187) (end 150.584927 111.331187) (width 0.25) (layer B.Cu) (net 13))
 (segment (start 126.708927 114.24426) (end 126.708927 115.649187) (width 0.25) (layer F.Cu) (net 13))
 (segment (start 119.223927 106.75926) (end 126.708927 114.24426) (width 0.25) (layer F.Cu) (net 13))
 (segment (start 119.20374 128.542374) (end 127.978927 119.767187) (width 0.25) (layer F.Cu) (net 13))
 (segment (start 119.20374 130.889187) (end 119.20374 128.542374) (width 0.25) (layer F.Cu) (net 13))
 (segment (start 79.00374 113.060114) (end 74.912927 108.969301) (width 1) (layer F.Cu) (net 14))
 (segment (start 74.912927 93.041187) (end 79.023927 88.930187) (width 1) (layer F.Cu) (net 14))
 (segment (start 74.912927 108.969301) (end 74.912927 93.041187) (width 1) (layer F.Cu) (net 14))
 (segment (start 79.00374 130.910114) (end 83.040927 126.872927) (width 1) (layer B.Cu) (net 15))
 (segment (start 83.040927 110.797187) (end 79.023927 106.780187) (width 1) (layer B.Cu) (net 15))
 (segment (start 83.040927 126.872927) (end 83.040927 110.797187) (width 1) (layer B.Cu) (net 15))
 (segment (start 128.113917 107.098197) (end 127.998927 107.213187) (width 0.25) (layer F.Cu) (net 8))
 (segment (start 126.728927 108.483187) (end 127.998927 107.213187) (width 0.25) (layer F.Cu) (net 8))
 (segment (start 126.728927 111.331187) (end 126.728927 108.483187) (width 0.25) (layer F.Cu) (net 8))
 (segment (start 127.998927 90.249187) (end 127.744927 89.995187) (width 0.25) (layer F.Cu) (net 8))
 (segment (start 127.998927 107.213187) (end 127.998927 90.249187) (width 0.25) (layer F.Cu) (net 8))
 (segment (start 138.686927 108.483187) (end 139.956927 107.213187) (width 0.25) (layer F.Cu) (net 9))
 (segment (start 138.686927 111.331187) (end 138.686927 108.483187) (width 0.25) (layer F.Cu) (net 9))
 (segment (start 135.110927 102.367187) (end 135.782927 103.039187) (width 0.25) (layer F.Cu) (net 9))
 (segment (start 135.782927 103.039187) (end 139.956927 107.213187) (width 0.25) (layer F.Cu) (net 9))
 (segment (start 135.618927 102.875187) (end 135.782927 103.039187) (width 0.25) (layer F.Cu) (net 9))
 (segment (start 135.110927 94.821187) (end 135.110927 102.367187) (width 0.25) (layer F.Cu) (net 9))
 (segment (start 130.284927 89.995187) (end 135.110927 94.821187) (width 0.25) (layer F.Cu) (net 9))
 (segment (start 144.996927 116.919187) (end 146.266927 115.649187) (width 0.25) (layer F.Cu) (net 10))
 (segment (start 144.996927 119.767187) (end 144.996927 116.919187) (width 0.25) (layer F.Cu) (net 10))
 (segment (start 147.556927 114.359187) (end 146.266927 115.649187) (width 0.25) (layer F.Cu) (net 10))
 (segment (start 147.556927 101.679187) (end 147.556927 114.359187) (width 0.25) (layer F.Cu) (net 10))
 (segment (start 143.365927 97.488187) (end 147.556927 101.679187) (width 0.25) (layer F.Cu) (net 10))
 (segment (start 140.317927 97.488187) (end 143.365927 97.488187) (width 0.25) (layer F.Cu) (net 10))
 (segment (start 132.824927 89.995187) (end 140.317927 97.488187) (width 0.25) (layer F.Cu) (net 10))
 (segment (start 148.318927 113.617187) (end 148.298927 113.617187) (width 0.25) (layer F.Cu) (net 11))
 (segment (start 133.058927 116.919187) (end 134.328927 115.649187) (width 0.25) (layer F.Cu) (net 11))
 (segment (start 133.058927 119.767187) (end 133.058927 116.919187) (width 0.25) (layer F.Cu) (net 11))
 (segment (start 135.364927 91.519187) (end 135.364927 89.995187) (width 0.25) (layer F.Cu) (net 11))
 (segment (start 140.508427 96.662687) (end 135.364927 91.519187) (width 0.25) (layer F.Cu) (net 11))
 (segment (start 148.318927 127.841187) (end 148.318927 101.552187) (width 0.25) (layer F.Cu) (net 11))
 (segment (start 148.318927 101.552187) (end 143.429427 96.662687) (width 0.25) (layer F.Cu) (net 11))
 (segment (start 143.746927 132.413187) (end 148.318927 127.841187) (width 0.25) (layer F.Cu) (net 11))
 (segment (start 143.429427 96.662687) (end 140.508427 96.662687) (width 0.25) (layer F.Cu) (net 11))
 (segment (start 139.428927 132.413187) (end 143.746927 132.413187) (width 0.25) (layer F.Cu) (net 11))
 (segment (start 136.126927 129.111187) (end 139.428927 132.413187) (width 0.25) (layer F.Cu) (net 11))
 (segment (start 136.126927 122.835187) (end 136.126927 129.111187) (width 0.25) (layer F.Cu) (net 11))
 (segment (start 133.058927 119.767187) (end 136.126927 122.835187) (width 0.25) (layer F.Cu) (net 11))
 (segment (start 164.574927 122.962187) (end 161.506927 119.894187) (width 0.25) (layer F.Cu) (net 4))
 (segment (start 164.574927 129.111187) (end 164.574927 122.962187) (width 0.25) (layer F.Cu) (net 4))
 (segment (start 172.448927 131.651187) (end 167.114927 131.651187) (width 0.25) (layer F.Cu) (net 4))
 (segment (start 178.036927 126.063187) (end 172.448927 131.651187) (width 0.25) (layer F.Cu) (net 4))
 (segment (start 167.114927 131.651187) (end 164.574927 129.111187) (width 0.25) (layer F.Cu) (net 4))
 (segment (start 162.776927 118.624187) (end 161.506927 119.894187) (width 0.25) (layer F.Cu) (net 4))
 (segment (start 162.776927 115.903187) (end 162.776927 118.624187) (width 0.25) (layer F.Cu) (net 4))
 (segment (start 178.036927 99.647187) (end 178.036927 126.063187) (width 0.25) (layer F.Cu) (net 4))
 (segment (start 172.702927 94.313187) (end 178.036927 99.647187) (width 0.25) (layer F.Cu) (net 4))
 (segment (start 172.702927 90.249187) (end 172.702927 94.313187) (width 0.25) (layer F.Cu) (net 4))
 (segment (start 174.714927 118.624187) (end 173.444927 119.894187) (width 0.25) (layer F.Cu) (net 5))
 (segment (start 174.714927 115.903187) (end 174.714927 118.624187) (width 0.25) (layer F.Cu) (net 5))
 (segment (start 176.258927 114.359187) (end 174.714927 115.903187) (width 0.25) (layer F.Cu) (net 5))
 (segment (start 176.258927 100.409187) (end 176.258927 114.359187) (width 0.25) (layer F.Cu) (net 5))
 (segment (start 170.162927 94.313187) (end 176.258927 100.409187) (width 0.25) (layer F.Cu) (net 5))
 (segment (start 170.162927 90.249187) (end 170.162927 94.313187) (width 0.25) (layer F.Cu) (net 5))
 (segment (start 167.114927 108.737187) (end 168.384927 107.467187) (width 0.25) (layer F.Cu) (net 6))
 (segment (start 167.114927 111.585187) (end 167.114927 108.737187) (width 0.25) (layer F.Cu) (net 6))
 (segment (start 168.384927 107.467187) (end 168.384927 107.267187) (width 0.25) (layer F.Cu) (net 6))
 (segment (start 168.384927 107.267187) (end 165.844927 104.727187) (width 0.25) (layer F.Cu) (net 6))
 (segment (start 165.844927 92.027187) (end 167.622927 90.249187) (width 0.25) (layer F.Cu) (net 6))
 (segment (start 165.844927 104.727187) (end 165.844927 92.027187) (width 0.25) (layer F.Cu) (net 6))
 (segment (start 155.196927 108.737187) (end 156.466927 107.467187) (width 0.25) (layer F.Cu) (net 7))
 (segment (start 155.196927 111.585187) (end 155.196927 108.737187) (width 0.25) (layer F.Cu) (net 7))
 (segment (start 156.581917 107.352197) (end 156.466927 107.467187) (width 0.25) (layer F.Cu) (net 7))
 (segment (start 165.082927 90.249187) (end 164.828927 90.249187) (width 0.25) (layer F.Cu) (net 7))
 (segment (start 156.581917 98.496197) (end 156.581917 99.020177) (width 0.25) (layer F.Cu) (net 7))
 (segment (start 164.828927 90.249187) (end 156.581917 98.496197) (width 0.25) (layer F.Cu) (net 7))
 (segment (start 156.581917 99.020177) (end 156.581917 107.352197) (width 0.25) (layer F.Cu) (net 7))
 (segment (start 148.298927 90.737187) (end 147.048927 89.487187) (width 0.25) (layer F.Cu) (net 1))
 (segment (start 148.298927 92.789187) (end 148.298927 90.737187) (width 0.25) (layer F.Cu) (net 1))
 (segment (start 146.540927 89.995187) (end 147.048927 89.487187) (width 0.25) (layer F.Cu) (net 1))
 (segment (start 143.492927 89.995187) (end 146.540927 89.995187) (width 0.25) (layer F.Cu) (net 1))
 (segment (start 143.492927 93.805187) (end 143.746927 93.805187) (width 0.25) (layer F.Cu) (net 3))
 (segment (start 143.746927 93.805187) (end 145.270927 95.329187) (width 0.25) (layer F.Cu) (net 3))
 (segment (start 150.838927 95.329187) (end 153.378927 92.789187) (width 0.25) (layer F.Cu) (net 3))
 (segment (start 145.270927 95.329187) (end 150.838927 95.329187) (width 0.25) (layer F.Cu) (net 3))
 (segment (start 153.378927 90.777187) (end 154.668927 89.487187) (width 0.25) (layer F.Cu) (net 3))
 (segment (start 153.378927 92.789187) (end 153.378927 90.777187) (width 0.25) (layer F.Cu) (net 3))
 (segment (start 158.224927 89.995187) (end 158.224927 89.487187) (width 0.25) (layer F.Cu) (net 2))
 (segment (start 158.224927 89.487187) (end 156.446927 87.709187) (width 0.25) (layer F.Cu) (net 2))
 (segment (start 152.088927 87.709187) (end 150.838927 88.959187) (width 0.25) (layer F.Cu) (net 2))
 (segment (start 156.446927 87.709187) (end 152.088927 87.709187) (width 0.25) (layer F.Cu) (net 2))
 (segment (start 150.838927 92.789187) (end 150.838927 88.959187) (width 0.25) (layer F.Cu) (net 2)))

